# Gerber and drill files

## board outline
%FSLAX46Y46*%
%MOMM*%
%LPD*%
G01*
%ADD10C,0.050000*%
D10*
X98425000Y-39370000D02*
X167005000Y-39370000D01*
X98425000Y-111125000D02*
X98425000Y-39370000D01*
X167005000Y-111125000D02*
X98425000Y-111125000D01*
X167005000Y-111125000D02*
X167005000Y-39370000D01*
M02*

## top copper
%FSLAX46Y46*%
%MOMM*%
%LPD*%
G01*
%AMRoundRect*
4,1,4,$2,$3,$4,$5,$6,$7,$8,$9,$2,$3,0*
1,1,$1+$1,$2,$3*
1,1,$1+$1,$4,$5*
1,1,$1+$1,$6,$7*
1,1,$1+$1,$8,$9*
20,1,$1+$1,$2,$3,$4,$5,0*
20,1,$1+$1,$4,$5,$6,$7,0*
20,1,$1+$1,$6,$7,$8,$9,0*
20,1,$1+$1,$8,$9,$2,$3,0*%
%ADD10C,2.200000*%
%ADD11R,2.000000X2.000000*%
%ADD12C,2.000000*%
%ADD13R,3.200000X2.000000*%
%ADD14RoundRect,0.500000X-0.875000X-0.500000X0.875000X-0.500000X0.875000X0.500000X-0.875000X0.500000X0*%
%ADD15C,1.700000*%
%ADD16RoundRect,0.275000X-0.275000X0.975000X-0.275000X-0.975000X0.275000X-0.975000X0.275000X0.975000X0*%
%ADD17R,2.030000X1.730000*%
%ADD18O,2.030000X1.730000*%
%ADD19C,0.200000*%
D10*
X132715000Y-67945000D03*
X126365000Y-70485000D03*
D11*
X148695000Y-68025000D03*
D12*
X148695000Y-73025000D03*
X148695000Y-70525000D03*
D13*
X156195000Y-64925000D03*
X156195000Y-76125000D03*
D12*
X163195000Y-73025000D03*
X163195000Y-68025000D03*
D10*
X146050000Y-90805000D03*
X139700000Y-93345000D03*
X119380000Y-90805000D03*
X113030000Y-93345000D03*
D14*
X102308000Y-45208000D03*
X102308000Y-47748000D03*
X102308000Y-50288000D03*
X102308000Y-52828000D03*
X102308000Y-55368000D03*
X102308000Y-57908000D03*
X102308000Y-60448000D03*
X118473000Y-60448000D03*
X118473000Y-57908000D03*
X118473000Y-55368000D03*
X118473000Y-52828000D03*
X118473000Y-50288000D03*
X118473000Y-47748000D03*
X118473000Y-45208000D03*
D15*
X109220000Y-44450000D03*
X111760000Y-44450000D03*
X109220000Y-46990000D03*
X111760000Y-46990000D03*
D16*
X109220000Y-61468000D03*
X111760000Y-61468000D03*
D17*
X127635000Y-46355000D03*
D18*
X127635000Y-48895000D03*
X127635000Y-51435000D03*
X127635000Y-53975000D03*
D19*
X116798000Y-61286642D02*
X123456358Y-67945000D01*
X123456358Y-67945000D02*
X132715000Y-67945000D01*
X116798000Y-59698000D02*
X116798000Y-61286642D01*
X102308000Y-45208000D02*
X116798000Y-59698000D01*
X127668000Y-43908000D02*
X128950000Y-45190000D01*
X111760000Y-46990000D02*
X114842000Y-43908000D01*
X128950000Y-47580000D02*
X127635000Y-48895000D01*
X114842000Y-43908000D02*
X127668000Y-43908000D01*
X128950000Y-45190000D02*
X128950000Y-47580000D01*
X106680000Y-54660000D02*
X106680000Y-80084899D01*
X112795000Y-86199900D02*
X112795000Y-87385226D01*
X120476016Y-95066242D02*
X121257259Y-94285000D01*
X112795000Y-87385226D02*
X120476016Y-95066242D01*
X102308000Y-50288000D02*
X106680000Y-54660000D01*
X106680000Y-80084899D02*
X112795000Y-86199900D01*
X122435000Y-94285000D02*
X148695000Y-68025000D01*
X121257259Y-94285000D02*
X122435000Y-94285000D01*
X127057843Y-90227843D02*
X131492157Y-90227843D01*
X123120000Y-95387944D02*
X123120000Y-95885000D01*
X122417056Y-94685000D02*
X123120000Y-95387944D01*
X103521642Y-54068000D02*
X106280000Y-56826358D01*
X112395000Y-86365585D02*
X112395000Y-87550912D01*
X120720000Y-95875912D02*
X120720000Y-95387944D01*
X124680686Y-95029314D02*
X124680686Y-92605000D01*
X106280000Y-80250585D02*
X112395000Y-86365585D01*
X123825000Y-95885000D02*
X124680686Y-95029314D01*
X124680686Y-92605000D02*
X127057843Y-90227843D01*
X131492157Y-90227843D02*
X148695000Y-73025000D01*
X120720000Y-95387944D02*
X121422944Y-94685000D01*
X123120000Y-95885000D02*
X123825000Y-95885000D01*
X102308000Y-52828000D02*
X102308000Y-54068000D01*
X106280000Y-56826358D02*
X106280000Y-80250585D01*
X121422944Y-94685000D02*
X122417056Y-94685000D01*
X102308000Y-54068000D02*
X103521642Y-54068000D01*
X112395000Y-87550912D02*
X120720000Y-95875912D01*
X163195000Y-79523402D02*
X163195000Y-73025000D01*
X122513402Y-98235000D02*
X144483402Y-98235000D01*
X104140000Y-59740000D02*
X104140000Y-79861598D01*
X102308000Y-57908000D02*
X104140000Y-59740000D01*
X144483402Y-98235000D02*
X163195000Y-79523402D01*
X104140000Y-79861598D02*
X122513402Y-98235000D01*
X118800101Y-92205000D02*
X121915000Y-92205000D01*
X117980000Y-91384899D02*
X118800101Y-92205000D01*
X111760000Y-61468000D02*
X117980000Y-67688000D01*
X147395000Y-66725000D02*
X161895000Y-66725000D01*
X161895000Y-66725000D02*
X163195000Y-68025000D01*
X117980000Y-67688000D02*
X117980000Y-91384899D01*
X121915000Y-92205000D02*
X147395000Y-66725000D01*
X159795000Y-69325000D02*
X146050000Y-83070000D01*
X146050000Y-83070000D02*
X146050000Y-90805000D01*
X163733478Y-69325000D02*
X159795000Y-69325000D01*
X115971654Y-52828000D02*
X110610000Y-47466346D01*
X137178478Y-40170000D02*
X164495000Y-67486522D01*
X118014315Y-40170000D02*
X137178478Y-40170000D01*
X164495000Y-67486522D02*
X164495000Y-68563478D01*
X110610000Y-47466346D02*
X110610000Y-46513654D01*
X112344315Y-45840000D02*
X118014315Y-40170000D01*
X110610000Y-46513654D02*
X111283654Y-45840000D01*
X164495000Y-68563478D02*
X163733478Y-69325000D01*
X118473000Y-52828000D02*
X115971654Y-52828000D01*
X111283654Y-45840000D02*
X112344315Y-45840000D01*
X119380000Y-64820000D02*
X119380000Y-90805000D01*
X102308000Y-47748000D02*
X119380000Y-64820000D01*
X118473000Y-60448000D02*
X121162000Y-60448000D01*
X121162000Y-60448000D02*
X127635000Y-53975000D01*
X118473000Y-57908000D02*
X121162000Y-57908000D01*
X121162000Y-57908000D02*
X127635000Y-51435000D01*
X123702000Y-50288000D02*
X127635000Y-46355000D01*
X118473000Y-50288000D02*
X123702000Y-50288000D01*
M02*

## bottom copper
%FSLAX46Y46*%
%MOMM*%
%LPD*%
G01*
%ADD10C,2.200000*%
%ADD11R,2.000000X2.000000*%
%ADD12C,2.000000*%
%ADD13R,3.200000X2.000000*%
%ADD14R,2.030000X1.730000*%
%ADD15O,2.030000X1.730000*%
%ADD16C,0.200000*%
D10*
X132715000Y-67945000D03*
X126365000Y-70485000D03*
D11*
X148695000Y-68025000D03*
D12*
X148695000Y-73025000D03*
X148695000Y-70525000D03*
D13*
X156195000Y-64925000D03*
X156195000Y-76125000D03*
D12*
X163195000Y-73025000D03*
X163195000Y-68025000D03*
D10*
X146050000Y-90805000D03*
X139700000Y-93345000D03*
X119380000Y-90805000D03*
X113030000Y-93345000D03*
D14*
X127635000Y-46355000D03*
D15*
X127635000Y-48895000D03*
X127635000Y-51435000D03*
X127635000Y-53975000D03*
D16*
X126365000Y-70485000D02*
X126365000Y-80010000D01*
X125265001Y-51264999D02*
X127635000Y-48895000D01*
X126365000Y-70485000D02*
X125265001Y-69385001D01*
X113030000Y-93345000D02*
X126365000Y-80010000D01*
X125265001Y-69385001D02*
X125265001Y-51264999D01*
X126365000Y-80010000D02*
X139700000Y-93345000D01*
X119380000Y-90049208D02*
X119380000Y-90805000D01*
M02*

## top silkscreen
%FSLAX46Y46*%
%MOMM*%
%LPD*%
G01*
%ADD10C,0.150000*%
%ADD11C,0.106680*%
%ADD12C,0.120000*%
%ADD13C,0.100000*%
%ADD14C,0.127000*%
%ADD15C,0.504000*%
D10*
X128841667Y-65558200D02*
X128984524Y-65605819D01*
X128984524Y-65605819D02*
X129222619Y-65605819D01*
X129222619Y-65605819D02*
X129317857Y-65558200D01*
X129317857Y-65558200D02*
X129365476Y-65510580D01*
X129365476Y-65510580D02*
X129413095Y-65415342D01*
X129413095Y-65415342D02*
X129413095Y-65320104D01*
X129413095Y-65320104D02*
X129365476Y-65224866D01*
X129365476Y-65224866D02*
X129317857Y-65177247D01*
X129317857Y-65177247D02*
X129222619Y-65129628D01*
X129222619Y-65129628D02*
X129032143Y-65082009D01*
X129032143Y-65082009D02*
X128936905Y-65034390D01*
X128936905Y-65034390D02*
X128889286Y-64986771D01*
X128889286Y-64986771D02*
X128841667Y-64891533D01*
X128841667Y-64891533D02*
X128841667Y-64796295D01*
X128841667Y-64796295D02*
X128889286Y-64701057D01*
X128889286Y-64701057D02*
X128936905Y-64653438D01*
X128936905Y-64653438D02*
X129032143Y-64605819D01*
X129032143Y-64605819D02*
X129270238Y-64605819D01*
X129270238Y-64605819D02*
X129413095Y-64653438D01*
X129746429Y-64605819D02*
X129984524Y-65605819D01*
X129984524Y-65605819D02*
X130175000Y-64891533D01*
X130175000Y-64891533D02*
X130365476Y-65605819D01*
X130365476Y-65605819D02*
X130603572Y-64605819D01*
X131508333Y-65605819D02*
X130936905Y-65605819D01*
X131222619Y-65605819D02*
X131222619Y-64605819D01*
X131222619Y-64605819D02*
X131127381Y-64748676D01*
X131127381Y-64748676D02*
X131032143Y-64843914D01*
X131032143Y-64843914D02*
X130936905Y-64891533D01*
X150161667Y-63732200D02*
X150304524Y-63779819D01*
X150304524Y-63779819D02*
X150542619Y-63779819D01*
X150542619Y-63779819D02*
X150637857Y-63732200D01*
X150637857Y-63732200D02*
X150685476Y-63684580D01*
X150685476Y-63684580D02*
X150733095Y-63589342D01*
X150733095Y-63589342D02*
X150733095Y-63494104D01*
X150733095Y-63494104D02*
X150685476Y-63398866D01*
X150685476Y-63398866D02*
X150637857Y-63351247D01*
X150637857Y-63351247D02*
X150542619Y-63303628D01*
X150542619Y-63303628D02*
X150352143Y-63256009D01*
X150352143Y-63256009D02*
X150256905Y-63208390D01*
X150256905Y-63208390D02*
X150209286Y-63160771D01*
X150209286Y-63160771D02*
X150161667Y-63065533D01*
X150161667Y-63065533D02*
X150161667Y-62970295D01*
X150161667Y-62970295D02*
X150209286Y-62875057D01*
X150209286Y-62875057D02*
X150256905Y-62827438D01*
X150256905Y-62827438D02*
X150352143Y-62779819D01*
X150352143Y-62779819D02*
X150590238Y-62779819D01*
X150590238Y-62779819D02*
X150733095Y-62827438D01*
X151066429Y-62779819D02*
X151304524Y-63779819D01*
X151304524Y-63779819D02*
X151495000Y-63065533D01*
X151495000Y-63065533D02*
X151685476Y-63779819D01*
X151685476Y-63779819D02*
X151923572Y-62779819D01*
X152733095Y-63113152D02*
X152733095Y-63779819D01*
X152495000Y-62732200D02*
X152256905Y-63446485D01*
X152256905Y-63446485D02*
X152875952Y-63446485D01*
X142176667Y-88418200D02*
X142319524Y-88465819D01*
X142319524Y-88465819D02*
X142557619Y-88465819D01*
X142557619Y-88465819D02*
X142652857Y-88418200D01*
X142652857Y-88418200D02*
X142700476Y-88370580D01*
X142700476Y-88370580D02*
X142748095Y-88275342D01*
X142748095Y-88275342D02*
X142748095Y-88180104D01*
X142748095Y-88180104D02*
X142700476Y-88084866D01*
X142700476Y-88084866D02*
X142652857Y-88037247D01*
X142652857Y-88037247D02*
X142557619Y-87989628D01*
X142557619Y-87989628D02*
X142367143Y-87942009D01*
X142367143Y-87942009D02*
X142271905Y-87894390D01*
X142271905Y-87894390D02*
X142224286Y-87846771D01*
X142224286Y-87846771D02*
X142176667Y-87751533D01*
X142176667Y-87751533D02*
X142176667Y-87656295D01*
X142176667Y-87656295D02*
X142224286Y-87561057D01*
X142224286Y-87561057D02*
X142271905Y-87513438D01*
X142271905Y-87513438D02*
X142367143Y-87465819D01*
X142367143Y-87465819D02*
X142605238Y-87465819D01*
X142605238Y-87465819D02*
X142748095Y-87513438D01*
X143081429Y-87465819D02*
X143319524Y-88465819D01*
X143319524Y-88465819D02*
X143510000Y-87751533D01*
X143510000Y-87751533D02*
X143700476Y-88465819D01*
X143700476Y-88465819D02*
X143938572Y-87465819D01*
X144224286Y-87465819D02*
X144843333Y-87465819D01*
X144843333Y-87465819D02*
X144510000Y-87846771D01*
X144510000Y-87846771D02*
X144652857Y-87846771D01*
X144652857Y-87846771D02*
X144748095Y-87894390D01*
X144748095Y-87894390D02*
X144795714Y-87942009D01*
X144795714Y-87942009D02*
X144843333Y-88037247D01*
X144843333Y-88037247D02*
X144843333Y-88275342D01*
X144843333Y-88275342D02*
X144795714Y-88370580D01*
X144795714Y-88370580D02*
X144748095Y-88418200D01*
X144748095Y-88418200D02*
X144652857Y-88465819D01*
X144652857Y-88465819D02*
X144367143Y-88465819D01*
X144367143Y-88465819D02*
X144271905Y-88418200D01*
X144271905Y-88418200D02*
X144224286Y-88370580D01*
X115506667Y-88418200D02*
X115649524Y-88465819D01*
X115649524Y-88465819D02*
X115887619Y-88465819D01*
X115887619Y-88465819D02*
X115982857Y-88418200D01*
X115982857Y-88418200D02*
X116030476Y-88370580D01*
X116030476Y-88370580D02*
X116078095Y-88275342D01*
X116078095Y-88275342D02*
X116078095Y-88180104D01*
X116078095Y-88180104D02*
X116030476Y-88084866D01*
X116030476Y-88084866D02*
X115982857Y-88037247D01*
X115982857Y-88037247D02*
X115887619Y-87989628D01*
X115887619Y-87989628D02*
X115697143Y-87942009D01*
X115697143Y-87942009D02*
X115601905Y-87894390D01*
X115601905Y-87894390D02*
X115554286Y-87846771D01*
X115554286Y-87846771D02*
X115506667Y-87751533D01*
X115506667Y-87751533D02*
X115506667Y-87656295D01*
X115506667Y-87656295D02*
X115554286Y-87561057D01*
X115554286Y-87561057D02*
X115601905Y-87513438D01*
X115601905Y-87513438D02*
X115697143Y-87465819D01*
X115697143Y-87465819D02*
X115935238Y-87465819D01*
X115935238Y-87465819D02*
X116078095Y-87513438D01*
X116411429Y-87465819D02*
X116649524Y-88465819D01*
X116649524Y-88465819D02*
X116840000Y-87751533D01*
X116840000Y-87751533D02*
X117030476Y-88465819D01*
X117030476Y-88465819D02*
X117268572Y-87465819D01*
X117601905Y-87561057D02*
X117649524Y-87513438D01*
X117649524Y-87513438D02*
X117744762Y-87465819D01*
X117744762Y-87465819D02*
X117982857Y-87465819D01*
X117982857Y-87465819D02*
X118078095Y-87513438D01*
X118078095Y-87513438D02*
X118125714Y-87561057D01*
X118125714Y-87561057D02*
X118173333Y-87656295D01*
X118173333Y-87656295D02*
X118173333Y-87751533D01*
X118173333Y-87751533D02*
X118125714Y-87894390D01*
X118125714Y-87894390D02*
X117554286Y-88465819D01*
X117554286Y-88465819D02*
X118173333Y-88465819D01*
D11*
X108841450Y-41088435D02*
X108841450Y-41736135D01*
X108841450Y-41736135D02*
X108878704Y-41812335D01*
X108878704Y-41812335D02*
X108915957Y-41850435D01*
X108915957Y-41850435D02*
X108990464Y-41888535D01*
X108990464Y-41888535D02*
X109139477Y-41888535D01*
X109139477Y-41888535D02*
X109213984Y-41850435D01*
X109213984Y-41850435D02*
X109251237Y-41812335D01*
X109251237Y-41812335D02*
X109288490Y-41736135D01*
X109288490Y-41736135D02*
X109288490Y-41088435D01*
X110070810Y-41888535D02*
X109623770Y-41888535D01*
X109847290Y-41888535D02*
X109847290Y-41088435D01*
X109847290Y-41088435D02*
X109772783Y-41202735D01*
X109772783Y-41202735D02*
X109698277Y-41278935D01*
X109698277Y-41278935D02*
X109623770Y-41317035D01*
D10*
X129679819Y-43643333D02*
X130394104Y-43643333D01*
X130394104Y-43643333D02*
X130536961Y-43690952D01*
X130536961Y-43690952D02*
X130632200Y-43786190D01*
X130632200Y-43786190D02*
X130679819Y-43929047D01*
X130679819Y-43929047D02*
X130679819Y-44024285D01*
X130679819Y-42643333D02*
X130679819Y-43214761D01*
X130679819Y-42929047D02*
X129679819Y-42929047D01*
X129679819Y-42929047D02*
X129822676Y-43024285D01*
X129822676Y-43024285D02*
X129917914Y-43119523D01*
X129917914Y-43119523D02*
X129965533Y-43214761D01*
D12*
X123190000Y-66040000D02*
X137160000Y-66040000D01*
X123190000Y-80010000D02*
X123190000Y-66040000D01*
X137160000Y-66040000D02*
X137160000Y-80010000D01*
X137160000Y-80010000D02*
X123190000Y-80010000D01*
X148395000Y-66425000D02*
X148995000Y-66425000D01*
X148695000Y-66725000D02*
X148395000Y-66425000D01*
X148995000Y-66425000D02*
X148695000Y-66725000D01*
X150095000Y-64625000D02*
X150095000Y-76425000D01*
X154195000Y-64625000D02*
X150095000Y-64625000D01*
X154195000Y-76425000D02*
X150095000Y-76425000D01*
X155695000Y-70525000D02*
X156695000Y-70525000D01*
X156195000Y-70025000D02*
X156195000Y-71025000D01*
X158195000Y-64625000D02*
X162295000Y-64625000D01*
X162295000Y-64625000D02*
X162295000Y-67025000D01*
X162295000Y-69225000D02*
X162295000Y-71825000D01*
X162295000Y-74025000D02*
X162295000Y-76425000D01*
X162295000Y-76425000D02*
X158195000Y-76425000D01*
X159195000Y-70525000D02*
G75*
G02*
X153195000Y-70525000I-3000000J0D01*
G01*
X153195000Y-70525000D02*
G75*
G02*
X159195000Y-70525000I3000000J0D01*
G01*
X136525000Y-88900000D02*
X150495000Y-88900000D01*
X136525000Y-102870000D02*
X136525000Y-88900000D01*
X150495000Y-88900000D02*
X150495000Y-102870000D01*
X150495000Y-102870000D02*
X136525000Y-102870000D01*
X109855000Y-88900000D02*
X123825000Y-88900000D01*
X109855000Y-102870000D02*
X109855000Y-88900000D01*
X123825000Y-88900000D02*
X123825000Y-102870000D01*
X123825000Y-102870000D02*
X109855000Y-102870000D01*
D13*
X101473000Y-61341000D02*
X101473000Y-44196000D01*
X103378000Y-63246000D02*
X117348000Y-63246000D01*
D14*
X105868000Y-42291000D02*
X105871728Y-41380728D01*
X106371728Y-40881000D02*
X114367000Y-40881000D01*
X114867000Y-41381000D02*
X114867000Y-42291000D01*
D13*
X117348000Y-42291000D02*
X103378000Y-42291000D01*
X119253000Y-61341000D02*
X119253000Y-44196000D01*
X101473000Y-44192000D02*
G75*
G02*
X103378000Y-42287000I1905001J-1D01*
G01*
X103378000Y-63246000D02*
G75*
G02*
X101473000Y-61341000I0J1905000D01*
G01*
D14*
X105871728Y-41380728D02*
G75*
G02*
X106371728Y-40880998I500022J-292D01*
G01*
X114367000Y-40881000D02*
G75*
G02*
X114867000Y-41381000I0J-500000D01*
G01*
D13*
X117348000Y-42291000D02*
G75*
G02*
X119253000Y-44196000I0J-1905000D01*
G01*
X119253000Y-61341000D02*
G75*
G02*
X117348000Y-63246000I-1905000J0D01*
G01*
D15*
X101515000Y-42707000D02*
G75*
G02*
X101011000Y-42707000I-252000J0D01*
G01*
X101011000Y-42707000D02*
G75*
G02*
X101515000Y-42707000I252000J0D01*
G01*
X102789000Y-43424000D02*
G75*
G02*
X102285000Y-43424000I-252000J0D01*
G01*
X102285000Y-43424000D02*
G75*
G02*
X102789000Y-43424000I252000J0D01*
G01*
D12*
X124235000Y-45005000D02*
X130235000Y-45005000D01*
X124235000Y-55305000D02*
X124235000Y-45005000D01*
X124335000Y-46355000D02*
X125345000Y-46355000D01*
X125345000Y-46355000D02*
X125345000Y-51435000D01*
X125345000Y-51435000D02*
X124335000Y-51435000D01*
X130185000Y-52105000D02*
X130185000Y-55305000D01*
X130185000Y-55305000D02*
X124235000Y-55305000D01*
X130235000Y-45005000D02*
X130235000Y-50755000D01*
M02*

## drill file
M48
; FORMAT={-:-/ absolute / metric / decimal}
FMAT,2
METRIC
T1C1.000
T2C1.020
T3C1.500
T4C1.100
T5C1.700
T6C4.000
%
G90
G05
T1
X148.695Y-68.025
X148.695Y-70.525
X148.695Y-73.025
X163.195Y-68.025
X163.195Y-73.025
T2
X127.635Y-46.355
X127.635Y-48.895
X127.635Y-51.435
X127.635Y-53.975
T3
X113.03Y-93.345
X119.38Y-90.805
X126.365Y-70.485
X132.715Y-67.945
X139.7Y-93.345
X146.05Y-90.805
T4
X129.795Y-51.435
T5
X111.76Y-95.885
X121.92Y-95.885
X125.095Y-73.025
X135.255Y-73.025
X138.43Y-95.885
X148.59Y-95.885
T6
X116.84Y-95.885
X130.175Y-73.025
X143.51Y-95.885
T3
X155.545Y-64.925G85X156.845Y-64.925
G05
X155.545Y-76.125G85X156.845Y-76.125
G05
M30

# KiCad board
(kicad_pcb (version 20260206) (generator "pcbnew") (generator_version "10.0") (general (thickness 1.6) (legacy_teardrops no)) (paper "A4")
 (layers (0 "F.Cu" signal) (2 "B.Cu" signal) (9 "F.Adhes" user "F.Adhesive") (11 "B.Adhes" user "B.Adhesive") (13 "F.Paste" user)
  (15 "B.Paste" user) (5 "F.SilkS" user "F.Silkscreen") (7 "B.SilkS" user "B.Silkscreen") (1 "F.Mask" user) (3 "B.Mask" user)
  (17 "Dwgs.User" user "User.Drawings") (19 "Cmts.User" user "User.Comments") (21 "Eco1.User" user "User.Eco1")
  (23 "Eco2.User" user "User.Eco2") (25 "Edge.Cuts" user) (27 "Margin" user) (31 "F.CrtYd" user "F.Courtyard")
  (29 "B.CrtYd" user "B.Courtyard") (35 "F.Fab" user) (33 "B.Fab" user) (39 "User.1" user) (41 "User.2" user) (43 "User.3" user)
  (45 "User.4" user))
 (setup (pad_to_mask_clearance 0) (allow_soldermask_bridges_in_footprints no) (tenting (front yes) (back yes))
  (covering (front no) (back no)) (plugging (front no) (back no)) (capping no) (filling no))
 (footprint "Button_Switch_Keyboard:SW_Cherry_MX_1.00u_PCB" (layer "F.Cu") (at 132.715 67.945)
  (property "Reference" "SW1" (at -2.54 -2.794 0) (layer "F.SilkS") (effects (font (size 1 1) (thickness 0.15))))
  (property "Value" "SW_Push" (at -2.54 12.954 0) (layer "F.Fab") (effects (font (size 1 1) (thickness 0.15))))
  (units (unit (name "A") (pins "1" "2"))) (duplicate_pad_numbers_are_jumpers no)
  (fp_line (start -9.525 -1.905) (end 4.445 -1.905) (stroke (width 0.12) (type solid)) (layer "F.SilkS"))
  (fp_line (start -9.525 12.065) (end -9.525 -1.905) (stroke (width 0.12) (type solid)) (layer "F.SilkS"))
  (fp_line (start 4.445 -1.905) (end 4.445 12.065) (stroke (width 0.12) (type solid)) (layer "F.SilkS"))
  (fp_line (start 4.445 12.065) (end -9.525 12.065) (stroke (width 0.12) (type solid)) (layer "F.SilkS"))
  (pad "" np_thru_hole circle (at -7.62 5.08) (size 1.7 1.7) (drill 1.7) (layers "*.Cu" "*.Mask"))
  (pad "" np_thru_hole circle (at -2.54 5.08) (size 4 4) (drill 4) (layers "*.Cu" "*.Mask"))
  (pad "" np_thru_hole circle (at 2.54 5.08) (size 1.7 1.7) (drill 1.7) (layers "*.Cu" "*.Mask"))
  (pad "1" thru_hole circle (at 0 0) (size 2.2 2.2) (drill 1.5) (layers "*.Cu" "*.Mask") (remove_unused_layers no) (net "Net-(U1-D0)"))
  (pad "2" thru_hole circle (at -6.35 2.54) (size 2.2 2.2) (drill 1.5) (layers "*.Cu" "*.Mask") (remove_unused_layers no)
   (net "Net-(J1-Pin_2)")))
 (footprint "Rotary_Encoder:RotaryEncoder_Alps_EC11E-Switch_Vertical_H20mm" (layer "F.Cu") (at 148.695 68.025)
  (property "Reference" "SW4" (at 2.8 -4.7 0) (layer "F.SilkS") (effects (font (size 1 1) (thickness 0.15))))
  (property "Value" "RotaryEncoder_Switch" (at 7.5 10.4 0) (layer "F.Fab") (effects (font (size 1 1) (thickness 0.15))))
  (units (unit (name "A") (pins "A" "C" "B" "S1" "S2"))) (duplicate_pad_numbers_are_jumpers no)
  (fp_line (start -0.3 -1.6) (end 0.3 -1.6) (stroke (width 0.12) (type solid)) (layer "F.SilkS"))
  (fp_line (start 0 -1.3) (end -0.3 -1.6) (stroke (width 0.12) (type solid)) (layer "F.SilkS"))
  (fp_line (start 0.3 -1.6) (end 0 -1.3) (stroke (width 0.12) (type solid)) (layer "F.SilkS"))
  (fp_line (start 1.4 -3.4) (end 1.4 8.4) (stroke (width 0.12) (type solid)) (layer "F.SilkS"))
  (fp_line (start 5.5 -3.4) (end 1.4 -3.4) (stroke (width 0.12) (type solid)) (layer "F.SilkS"))
  (fp_line (start 5.5 8.4) (end 1.4 8.4) (stroke (width 0.12) (type solid)) (layer "F.SilkS"))
  (fp_line (start 7 2.5) (end 8 2.5) (stroke (width 0.12) (type solid)) (layer "F.SilkS"))
  (fp_line (start 7.5 2) (end 7.5 3) (stroke (width 0.12) (type solid)) (layer "F.SilkS"))
  (fp_line (start 9.5 -3.4) (end 13.6 -3.4) (stroke (width 0.12) (type solid)) (layer "F.SilkS"))
  (fp_line (start 13.6 -3.4) (end 13.6 -1) (stroke (width 0.12) (type solid)) (layer "F.SilkS"))
  (fp_line (start 13.6 1.2) (end 13.6 3.8) (stroke (width 0.12) (type solid)) (layer "F.SilkS"))
  (fp_line (start 13.6 6) (end 13.6 8.4) (stroke (width 0.12) (type solid)) (layer "F.SilkS"))
  (fp_line (start 13.6 8.4) (end 9.5 8.4) (stroke (width 0.12) (type solid)) (layer "F.SilkS"))
  (fp_circle (center 7.5 2.5) (end 10.5 2.5) (stroke (width 0.12) (type solid)) (fill no) (layer "F.SilkS"))
  (pad "A" thru_hole rect (at 0 0) (size 2 2) (drill 1) (layers "*.Cu" "*.Mask") (remove_unused_layers no) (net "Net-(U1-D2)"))
  (pad "B" thru_hole circle (at 0 5) (size 2 2) (drill 1) (layers "*.Cu" "*.Mask") (remove_unused_layers no) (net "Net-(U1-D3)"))
  (pad "C" thru_hole circle (at 0 2.5) (size 2 2) (drill 1) (layers "*.Cu" "*.Mask") (remove_unused_layers no)
   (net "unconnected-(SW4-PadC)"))
  (pad "MP" thru_hole rect (at 7.5 -3.1) (size 3.2 2) (drill oval 2.8 1.5) (layers "*.Cu" "*.Mask") (remove_unused_layers no))
  (pad "MP" thru_hole rect (at 7.5 8.1) (size 3.2 2) (drill oval 2.8 1.5) (layers "*.Cu" "*.Mask") (remove_unused_layers no))
  (pad "S1" thru_hole circle (at 14.5 5) (size 2 2) (drill 1) (layers "*.Cu" "*.Mask") (remove_unused_layers no) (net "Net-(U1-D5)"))
  (pad "S2" thru_hole circle (at 14.5 0) (size 2 2) (drill 1) (layers "*.Cu" "*.Mask") (remove_unused_layers no) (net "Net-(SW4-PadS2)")))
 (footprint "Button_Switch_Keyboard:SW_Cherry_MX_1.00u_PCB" (layer "F.Cu") (at 146.05 90.805)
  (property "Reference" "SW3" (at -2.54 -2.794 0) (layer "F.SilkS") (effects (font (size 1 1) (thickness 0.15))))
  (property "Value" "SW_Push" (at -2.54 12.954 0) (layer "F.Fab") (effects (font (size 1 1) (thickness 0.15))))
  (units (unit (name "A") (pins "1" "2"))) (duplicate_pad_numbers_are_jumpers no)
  (fp_line (start -9.525 -1.905) (end 4.445 -1.905) (stroke (width 0.12) (type solid)) (layer "F.SilkS"))
  (fp_line (start -9.525 12.065) (end -9.525 -1.905) (stroke (width 0.12) (type solid)) (layer "F.SilkS"))
  (fp_line (start 4.445 -1.905) (end 4.445 12.065) (stroke (width 0.12) (type solid)) (layer "F.SilkS"))
  (fp_line (start 4.445 12.065) (end -9.525 12.065) (stroke (width 0.12) (type solid)) (layer "F.SilkS"))
  (pad "" np_thru_hole circle (at -7.62 5.08) (size 1.7 1.7) (drill 1.7) (layers "*.Cu" "*.Mask"))
  (pad "" np_thru_hole circle (at -2.54 5.08) (size 4 4) (drill 4) (layers "*.Cu" "*.Mask"))
  (pad "" np_thru_hole circle (at 2.54 5.08) (size 1.7 1.7) (drill 1.7) (layers "*.Cu" "*.Mask"))
  (pad "1" thru_hole circle (at 0 0) (size 2.2 2.2) (drill 1.5) (layers "*.Cu" "*.Mask") (remove_unused_layers no) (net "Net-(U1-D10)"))
  (pad "2" thru_hole circle (at -6.35 2.54) (size 2.2 2.2) (drill 1.5) (layers "*.Cu" "*.Mask") (remove_unused_layers no)
   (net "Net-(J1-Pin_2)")))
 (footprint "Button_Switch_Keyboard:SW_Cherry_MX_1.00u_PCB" (layer "F.Cu") (at 119.38 90.805)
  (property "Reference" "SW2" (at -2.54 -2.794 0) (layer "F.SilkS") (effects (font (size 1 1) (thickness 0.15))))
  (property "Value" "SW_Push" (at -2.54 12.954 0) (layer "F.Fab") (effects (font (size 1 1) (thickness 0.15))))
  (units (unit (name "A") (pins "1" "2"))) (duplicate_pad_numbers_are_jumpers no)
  (fp_line (start -9.525 -1.905) (end 4.445 -1.905) (stroke (width 0.12) (type solid)) (layer "F.SilkS"))
  (fp_line (start -9.525 12.065) (end -9.525 -1.905) (stroke (width 0.12) (type solid)) (layer "F.SilkS"))
  (fp_line (start 4.445 -1.905) (end 4.445 12.065) (stroke (width 0.12) (type solid)) (layer "F.SilkS"))
  (fp_line (start 4.445 12.065) (end -9.525 12.065) (stroke (width 0.12) (type solid)) (layer "F.SilkS"))
  (pad "" np_thru_hole circle (at -7.62 5.08) (size 1.7 1.7) (drill 1.7) (layers "*.Cu" "*.Mask"))
  (pad "" np_thru_hole circle (at -2.54 5.08) (size 4 4) (drill 4) (layers "*.Cu" "*.Mask"))
  (pad "" np_thru_hole circle (at 2.54 5.08) (size 1.7 1.7) (drill 1.7) (layers "*.Cu" "*.Mask"))
  (pad "1" thru_hole circle (at 0 0) (size 2.2 2.2) (drill 1.5) (layers "*.Cu" "*.Mask") (remove_unused_layers no) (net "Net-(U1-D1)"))
  (pad "2" thru_hole circle (at -6.35 2.54) (size 2.2 2.2) (drill 1.5) (layers "*.Cu" "*.Mask") (remove_unused_layers no)
   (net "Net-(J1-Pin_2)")))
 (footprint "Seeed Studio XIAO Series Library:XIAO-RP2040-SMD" (layer "F.Cu") (at 101.473 63.328)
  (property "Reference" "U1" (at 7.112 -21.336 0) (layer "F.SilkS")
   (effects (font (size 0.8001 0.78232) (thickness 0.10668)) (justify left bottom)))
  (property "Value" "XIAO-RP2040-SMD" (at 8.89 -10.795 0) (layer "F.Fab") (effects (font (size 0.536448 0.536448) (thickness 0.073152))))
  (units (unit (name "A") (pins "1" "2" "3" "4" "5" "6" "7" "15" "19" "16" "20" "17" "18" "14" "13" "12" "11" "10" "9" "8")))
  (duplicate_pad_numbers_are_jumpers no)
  (fp_line (start 0 -1.987) (end 0 -19.132) (stroke (width 0.1) (type solid)) (layer "F.SilkS"))
  (fp_line (start 1.905 -0.082) (end 15.875 -0.082) (stroke (width 0.1) (type solid)) (layer "F.SilkS"))
  (fp_line (start 4.395 -21.037) (end 4.398728 -21.947272) (stroke (width 0.127) (type solid)) (layer "F.SilkS"))
  (fp_line (start 4.898728 -22.447) (end 12.894 -22.447) (stroke (width 0.127) (type solid)) (layer "F.SilkS"))
  (fp_line (start 13.394 -21.947) (end 13.394 -21.037) (stroke (width 0.127) (type solid)) (layer "F.SilkS"))
  (fp_line (start 15.875 -21.037) (end 1.905 -21.037) (stroke (width 0.1) (type solid)) (layer "F.SilkS"))
  (fp_line (start 17.78 -1.987) (end 17.78 -19.132) (stroke (width 0.1) (type solid)) (layer "F.SilkS"))
  (fp_arc (start 0 -19.136) (mid 0.557962 -20.483038) (end 1.905 -21.041) (stroke (width 0.1) (type solid)) (layer "F.SilkS"))
  (fp_arc (start 1.905 -0.082) (mid 0.557962 -0.639962) (end 0 -1.987) (stroke (width 0.1) (type solid)) (layer "F.SilkS"))
  (fp_arc (start 4.398728 -21.947272) (mid 4.545276 -22.300644) (end 4.898728 -22.447) (stroke (width 0.127) (type default))
   (layer "F.SilkS"))
  (fp_arc (start 12.894 -22.447) (mid 13.247553 -22.300553) (end 13.394 -21.947) (stroke (width 0.127) (type default)) (layer "F.SilkS"))
  (fp_arc (start 15.875 -21.037) (mid 17.222038 -20.479038) (end 17.78 -19.132) (stroke (width 0.1) (type solid)) (layer "F.SilkS"))
  (fp_arc (start 17.78 -1.987) (mid 17.222038 -0.639962) (end 15.875 -0.082) (stroke (width 0.1) (type solid)) (layer "F.SilkS"))
  (fp_circle (center -0.21 -20.621) (end -0.21 -20.875) (stroke (width 0.5) (type solid)) (fill yes) (layer "F.SilkS"))
  (fp_circle (center 1.064 -19.904) (end 1.064 -20.158) (stroke (width 0.5) (type solid)) (fill yes) (layer "F.SilkS"))
  (pad "1" smd roundrect (at 0.835 -18.12) (size 2.75 2) (layers "F.Cu" "F.Mask" "F.Paste") (roundrect_rratio 0.25) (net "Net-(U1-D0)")
   (solder_mask_margin 0.0508) (thermal_bridge_angle 45))
  (pad "2" smd roundrect (at 0.835 -15.58) (size 2.75 2) (layers "F.Cu" "F.Mask" "F.Paste") (roundrect_rratio 0.25) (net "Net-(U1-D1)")
   (solder_mask_margin 0.0508) (thermal_bridge_angle 45))
  (pad "3" smd roundrect (at 0.835 -13.04) (size 2.75 2) (layers "F.Cu" "F.Mask" "F.Paste") (roundrect_rratio 0.25) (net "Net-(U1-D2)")
   (solder_mask_margin 0.0508) (thermal_bridge_angle 45))
  (pad "4" smd roundrect (at 0.835 -10.5) (size 2.75 2) (layers "F.Cu" "F.Mask" "F.Paste") (roundrect_rratio 0.25) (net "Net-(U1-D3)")
   (solder_mask_margin 0.0508) (thermal_bridge_angle 45))
  (pad "5" smd roundrect (at 0.835 -7.96) (size 2.75 2) (layers "F.Cu" "F.Mask" "F.Paste") (roundrect_rratio 0.25)
   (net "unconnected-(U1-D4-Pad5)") (solder_mask_margin 0.0508) (thermal_bridge_angle 45))
  (pad "6" smd roundrect (at 0.835 -5.42) (size 2.75 2) (layers "F.Cu" "F.Mask" "F.Paste") (roundrect_rratio 0.25) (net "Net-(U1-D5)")
   (solder_mask_margin 0.0508) (thermal_bridge_angle 45))
  (pad "7" smd roundrect (at 0.835 -2.88) (size 2.75 2) (layers "F.Cu" "F.Mask" "F.Paste") (roundrect_rratio 0.25)
   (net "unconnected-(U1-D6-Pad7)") (solder_mask_margin 0.0508) (thermal_bridge_angle 45))
  (pad "8" smd roundrect (at 17 -2.88) (size 2.75 2) (layers "F.Cu" "F.Mask" "F.Paste") (roundrect_rratio 0.25) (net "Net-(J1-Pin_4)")
   (solder_mask_margin 0.0508) (thermal_bridge_angle 45))
  (pad "9" smd roundrect (at 17 -5.42) (size 2.75 2) (layers "F.Cu" "F.Mask" "F.Paste") (roundrect_rratio 0.25) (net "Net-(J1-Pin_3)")
   (solder_mask_margin 0.0508) (thermal_bridge_angle 45))
  (pad "10" smd roundrect (at 17 -7.96) (size 2.75 2) (layers "F.Cu" "F.Mask" "F.Paste") (roundrect_rratio 0.25)
   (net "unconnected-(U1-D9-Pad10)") (solder_mask_margin 0.0508) (thermal_bridge_angle 45))
  (pad "11" smd roundrect (at 17 -10.5) (size 2.75 2) (layers "F.Cu" "F.Mask" "F.Paste") (roundrect_rratio 0.25) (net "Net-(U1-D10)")
   (solder_mask_margin 0.0508) (thermal_bridge_angle 45))
  (pad "12" smd roundrect (at 17 -13.04) (size 2.75 2) (layers "F.Cu" "F.Mask" "F.Paste") (roundrect_rratio 0.25) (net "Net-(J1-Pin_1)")
   (solder_mask_margin 0.0508) (thermal_bridge_angle 45))
  (pad "13" smd roundrect (at 17 -15.58) (size 2.75 2) (layers "F.Cu" "F.Mask" "F.Paste") (roundrect_rratio 0.25)
   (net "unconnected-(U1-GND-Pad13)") (solder_mask_margin 0.0508) (thermal_bridge_angle 45))
  (pad "14" smd roundrect (at 17 -18.12) (size 2.75 2) (layers "F.Cu" "F.Mask" "F.Paste") (roundrect_rratio 0.25)
   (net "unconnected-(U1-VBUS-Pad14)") (solder_mask_margin 0.0508) (thermal_bridge_angle 45))
  (pad "15" smd circle (at 7.747 -18.878) (size 1.7 1.7) (layers "F.Cu" "F.Mask" "F.Paste") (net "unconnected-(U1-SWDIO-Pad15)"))
  (pad "16" smd circle (at 10.287 -18.878) (size 1.7 1.7) (layers "F.Cu" "F.Mask" "F.Paste") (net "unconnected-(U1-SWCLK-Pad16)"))
  (pad "17" smd circle (at 7.747 -16.338) (size 1.7 1.7) (layers "F.Cu" "F.Mask" "F.Paste") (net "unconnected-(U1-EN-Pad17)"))
  (pad "18" smd circle (at 10.287 -16.338) (size 1.7 1.7) (layers "F.Cu" "F.Mask" "F.Paste") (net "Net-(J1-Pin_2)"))
  (pad "19" smd roundrect (at 7.747 -1.86 270) (size 2.5 1.1) (layers "F.Cu" "F.Mask" "F.Paste") (roundrect_rratio 0.25)
   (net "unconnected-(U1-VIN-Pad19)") (thermal_bridge_angle 45))
  (pad "20" smd roundrect (at 10.287 -1.86 270) (size 2.5 1.1) (layers "F.Cu" "F.Mask" "F.Paste") (roundrect_rratio 0.25)
   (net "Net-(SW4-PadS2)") (thermal_bridge_angle 45)))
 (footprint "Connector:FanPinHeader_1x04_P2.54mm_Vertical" (layer "F.Cu") (at 127.635 46.355 -90)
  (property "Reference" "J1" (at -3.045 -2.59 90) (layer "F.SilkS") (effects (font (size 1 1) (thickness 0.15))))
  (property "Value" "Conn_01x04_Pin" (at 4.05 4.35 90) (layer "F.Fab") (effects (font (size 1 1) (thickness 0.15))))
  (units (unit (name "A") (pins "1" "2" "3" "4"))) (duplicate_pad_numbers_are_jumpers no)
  (fp_line (start -1.35 3.4) (end -1.35 -2.6) (stroke (width 0.12) (type solid)) (layer "F.SilkS"))
  (fp_line (start 8.95 3.4) (end -1.35 3.4) (stroke (width 0.12) (type solid)) (layer "F.SilkS"))
  (fp_line (start 0 3.3) (end 0 2.29) (stroke (width 0.12) (type solid)) (layer "F.SilkS"))
  (fp_line (start 0 2.29) (end 5.08 2.29) (stroke (width 0.12) (type solid)) (layer "F.SilkS"))
  (fp_line (start 5.08 2.29) (end 5.08 3.3) (stroke (width 0.12) (type solid)) (layer "F.SilkS"))
  (fp_line (start 5.75 -2.55) (end 8.95 -2.55) (stroke (width 0.12) (type solid)) (layer "F.SilkS"))
  (fp_line (start 8.95 -2.55) (end 8.95 3.4) (stroke (width 0.12) (type solid)) (layer "F.SilkS"))
  (fp_line (start -1.35 -2.6) (end 4.4 -2.6) (stroke (width 0.12) (type solid)) (layer "F.SilkS"))
  (pad "" np_thru_hole circle (at 5.08 -2.16) (size 1.1 1.1) (drill 1.1) (layers "*.Cu" "*.Mask"))
  (pad "1" thru_hole rect (at 0 0) (size 2.03 1.73) (drill 1.02) (layers "*.Cu" "*.Mask") (remove_unused_layers no) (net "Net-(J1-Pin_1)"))
  (pad "2" thru_hole oval (at 2.54 0) (size 2.03 1.73) (drill 1.02) (layers "*.Cu" "*.Mask") (remove_unused_layers no)
   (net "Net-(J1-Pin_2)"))
  (pad "3" thru_hole oval (at 5.08 0) (size 2.03 1.73) (drill 1.02) (layers "*.Cu" "*.Mask") (remove_unused_layers no)
   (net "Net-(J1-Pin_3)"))
  (pad "4" thru_hole oval (at 7.62 0) (size 2.03 1.73) (drill 1.02) (layers "*.Cu" "*.Mask") (remove_unused_layers no)
   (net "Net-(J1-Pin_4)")))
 (gr_line (start 98.425 39.37) (end 167.005 39.37) (stroke (width 0.05) (type default)) (layer "Edge.Cuts"))
 (gr_line (start 98.425 111.125) (end 98.425 39.37) (stroke (width 0.05) (type default)) (layer "Edge.Cuts"))
 (gr_line (start 167.005 111.125) (end 98.425 111.125) (stroke (width 0.05) (type default)) (layer "Edge.Cuts"))
 (gr_line (start 167.005 111.125) (end 167.005 39.37) (stroke (width 0.05) (type default)) (layer "Edge.Cuts"))
 (segment (start 116.798 61.286642) (end 123.456358 67.945) (width 0.2) (layer "F.Cu") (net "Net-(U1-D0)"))
 (segment (start 123.456358 67.945) (end 132.715 67.945) (width 0.2) (layer "F.Cu") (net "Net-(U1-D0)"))
 (segment (start 116.798 59.698) (end 116.798 61.286642) (width 0.2) (layer "F.Cu") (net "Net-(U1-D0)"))
 (segment (start 102.308 45.208) (end 116.798 59.698) (width 0.2) (layer "F.Cu") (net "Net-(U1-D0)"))
 (segment (start 127.668 43.908) (end 128.95 45.19) (width 0.2) (layer "F.Cu") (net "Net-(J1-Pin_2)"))
 (segment (start 111.76 46.99) (end 114.842 43.908) (width 0.2) (layer "F.Cu") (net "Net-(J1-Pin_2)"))
 (segment (start 128.95 47.58) (end 127.635 48.895) (width 0.2) (layer "F.Cu") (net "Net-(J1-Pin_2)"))
 (segment (start 114.842 43.908) (end 127.668 43.908) (width 0.2) (layer "F.Cu") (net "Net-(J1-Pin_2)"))
 (segment (start 128.95 45.19) (end 128.95 47.58) (width 0.2) (layer "F.Cu") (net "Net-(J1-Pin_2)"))
 (segment (start 126.365 70.485) (end 126.365 80.01) (width 0.2) (layer "B.Cu") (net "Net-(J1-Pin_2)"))
 (segment (start 125.265001 51.264999) (end 127.635 48.895) (width 0.2) (layer "B.Cu") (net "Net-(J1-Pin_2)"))
 (segment (start 126.365 70.485) (end 125.265001 69.385001) (width 0.2) (layer "B.Cu") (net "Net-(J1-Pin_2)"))
 (segment (start 113.03 93.345) (end 126.365 80.01) (width 0.2) (layer "B.Cu") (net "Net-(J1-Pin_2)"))
 (segment (start 125.265001 69.385001) (end 125.265001 51.264999) (width 0.2) (layer "B.Cu") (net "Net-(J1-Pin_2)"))
 (segment (start 126.365 80.01) (end 139.7 93.345) (width 0.2) (layer "B.Cu") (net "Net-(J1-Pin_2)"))
 (segment (start 106.68 54.66) (end 106.68 80.084899) (width 0.2) (layer "F.Cu") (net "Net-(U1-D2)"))
 (segment (start 112.795 86.1999) (end 112.795 87.385226) (width 0.2) (layer "F.Cu") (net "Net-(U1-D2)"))
 (segment (start 120.476016 95.066242) (end 121.257259 94.285) (width 0.2) (layer "F.Cu") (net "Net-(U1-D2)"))
 (segment (start 112.795 87.385226) (end 120.476016 95.066242) (width 0.2) (layer "F.Cu") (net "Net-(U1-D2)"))
 (segment (start 102.308 50.288) (end 106.68 54.66) (width 0.2) (layer "F.Cu") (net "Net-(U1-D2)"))
 (segment (start 106.68 80.084899) (end 112.795 86.1999) (width 0.2) (layer "F.Cu") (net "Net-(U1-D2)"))
 (segment (start 122.435 94.285) (end 148.695 68.025) (width 0.2) (layer "F.Cu") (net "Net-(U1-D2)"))
 (segment (start 121.257259 94.285) (end 122.435 94.285) (width 0.2) (layer "F.Cu") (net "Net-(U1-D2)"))
 (segment (start 127.057843 90.227843) (end 131.492157 90.227843) (width 0.2) (layer "F.Cu") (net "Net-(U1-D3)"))
 (segment (start 123.12 95.387944) (end 123.12 95.885) (width 0.2) (layer "F.Cu") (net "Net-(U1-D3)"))
 (segment (start 122.417056 94.685) (end 123.12 95.387944) (width 0.2) (layer "F.Cu") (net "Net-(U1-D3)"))
 (segment (start 103.521642 54.068) (end 106.28 56.826358) (width 0.2) (layer "F.Cu") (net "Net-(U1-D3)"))
 (segment (start 112.395 86.365585) (end 112.395 87.550912) (width 0.2) (layer "F.Cu") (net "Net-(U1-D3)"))
 (segment (start 120.72 95.875912) (end 120.72 95.387944) (width 0.2) (layer "F.Cu") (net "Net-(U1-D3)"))
 (segment (start 124.680686 95.029314) (end 124.680686 92.605) (width 0.2) (layer "F.Cu") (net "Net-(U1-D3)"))
 (segment (start 106.28 80.250585) (end 112.395 86.365585) (width 0.2) (layer "F.Cu") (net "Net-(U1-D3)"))
 (segment (start 123.825 95.885) (end 124.680686 95.029314) (width 0.2) (layer "F.Cu") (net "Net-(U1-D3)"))
 (segment (start 124.680686 92.605) (end 127.057843 90.227843) (width 0.2) (layer "F.Cu") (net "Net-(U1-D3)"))
 (segment (start 131.492157 90.227843) (end 148.695 73.025) (width 0.2) (layer "F.Cu") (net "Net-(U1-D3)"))
 (segment (start 120.72 95.387944) (end 121.422944 94.685) (width 0.2) (layer "F.Cu") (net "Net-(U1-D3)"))
 (segment (start 123.12 95.885) (end 123.825 95.885) (width 0.2) (layer "F.Cu") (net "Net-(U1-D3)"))
 (segment (start 102.308 52.828) (end 102.308 54.068) (width 0.2) (layer "F.Cu") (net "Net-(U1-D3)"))
 (segment (start 106.28 56.826358) (end 106.28 80.250585) (width 0.2) (layer "F.Cu") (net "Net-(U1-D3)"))
 (segment (start 121.422944 94.685) (end 122.417056 94.685) (width 0.2) (layer "F.Cu") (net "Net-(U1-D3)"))
 (segment (start 102.308 54.068) (end 103.521642 54.068) (width 0.2) (layer "F.Cu") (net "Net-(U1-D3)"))
 (segment (start 112.395 87.550912) (end 120.72 95.875912) (width 0.2) (layer "F.Cu") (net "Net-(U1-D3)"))
 (segment (start 163.195 79.523402) (end 163.195 73.025) (width 0.2) (layer "F.Cu") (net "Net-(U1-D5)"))
 (segment (start 122.513402 98.235) (end 144.483402 98.235) (width 0.2) (layer "F.Cu") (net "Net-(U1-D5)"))
 (segment (start 104.14 59.74) (end 104.14 79.861598) (width 0.2) (layer "F.Cu") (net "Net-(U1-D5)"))
 (segment (start 102.308 57.908) (end 104.14 59.74) (width 0.2) (layer "F.Cu") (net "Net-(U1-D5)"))
 (segment (start 144.483402 98.235) (end 163.195 79.523402) (width 0.2) (layer "F.Cu") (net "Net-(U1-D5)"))
 (segment (start 104.14 79.861598) (end 122.513402 98.235) (width 0.2) (layer "F.Cu") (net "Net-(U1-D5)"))
 (segment (start 118.800101 92.205) (end 121.915 92.205) (width 0.2) (layer "F.Cu") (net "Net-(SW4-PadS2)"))
 (segment (start 117.98 91.384899) (end 118.800101 92.205) (width 0.2) (layer "F.Cu") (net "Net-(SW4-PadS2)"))
 (segment (start 111.76 61.468) (end 117.98 67.688) (width 0.2) (layer "F.Cu") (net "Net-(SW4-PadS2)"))
 (segment (start 147.395 66.725) (end 161.895 66.725) (width 0.2) (layer "F.Cu") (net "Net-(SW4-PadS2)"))
 (segment (start 161.895 66.725) (end 163.195 68.025) (width 0.2) (layer "F.Cu") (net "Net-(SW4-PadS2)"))
 (segment (start 117.98 67.688) (end 117.98 91.384899) (width 0.2) (layer "F.Cu") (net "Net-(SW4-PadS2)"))
 (segment (start 121.915 92.205) (end 147.395 66.725) (width 0.2) (layer "F.Cu") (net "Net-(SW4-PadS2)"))
 (segment (start 159.795 69.325) (end 146.05 83.07) (width 0.2) (layer "F.Cu") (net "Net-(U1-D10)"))
 (segment (start 146.05 83.07) (end 146.05 90.805) (width 0.2) (layer "F.Cu") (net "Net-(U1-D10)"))
 (segment (start 163.733478 69.325) (end 159.795 69.325) (width 0.2) (layer "F.Cu") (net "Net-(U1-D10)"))
 (segment (start 115.971654 52.828) (end 110.61 47.466346) (width 0.2) (layer "F.Cu") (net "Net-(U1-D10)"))
 (segment (start 137.178478 40.17) (end 164.495 67.486522) (width 0.2) (layer "F.Cu") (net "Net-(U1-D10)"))
 (segment (start 118.014315 40.17) (end 137.178478 40.17) (width 0.2) (layer "F.Cu") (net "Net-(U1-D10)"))
 (segment (start 164.495 67.486522) (end 164.495 68.563478) (width 0.2) (layer "F.Cu") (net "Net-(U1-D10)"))
 (segment (start 110.61 47.466346) (end 110.61 46.513654) (width 0.2) (layer "F.Cu") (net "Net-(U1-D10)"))
 (segment (start 112.344315 45.84) (end 118.014315 40.17) (width 0.2) (layer "F.Cu") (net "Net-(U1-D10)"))
 (segment (start 110.61 46.513654) (end 111.283654 45.84) (width 0.2) (layer "F.Cu") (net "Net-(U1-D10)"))
 (segment (start 164.495 68.563478) (end 163.733478 69.325) (width 0.2) (layer "F.Cu") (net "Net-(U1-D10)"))
 (segment (start 118.473 52.828) (end 115.971654 52.828) (width 0.2) (layer "F.Cu") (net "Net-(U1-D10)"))
 (segment (start 111.283654 45.84) (end 112.344315 45.84) (width 0.2) (layer "F.Cu") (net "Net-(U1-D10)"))
 (segment (start 119.38 64.82) (end 119.38 90.805) (width 0.2) (layer "F.Cu") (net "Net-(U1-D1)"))
 (segment (start 102.308 47.748) (end 119.38 64.82) (width 0.2) (layer "F.Cu") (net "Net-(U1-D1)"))
 (segment (start 119.38 90.049208) (end 119.38 90.805) (width 0.2) (layer "B.Cu") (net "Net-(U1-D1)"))
 (segment (start 118.473 60.448) (end 121.162 60.448) (width 0.2) (layer "F.Cu") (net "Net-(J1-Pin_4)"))
 (segment (start 121.162 60.448) (end 127.635 53.975) (width 0.2) (layer "F.Cu") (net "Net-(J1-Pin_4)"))
 (segment (start 118.473 57.908) (end 121.162 57.908) (width 0.2) (layer "F.Cu") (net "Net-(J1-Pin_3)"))
 (segment (start 121.162 57.908) (end 127.635 51.435) (width 0.2) (layer "F.Cu") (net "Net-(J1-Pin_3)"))
 (segment (start 123.702 50.288) (end 127.635 46.355) (width 0.2) (layer "F.Cu") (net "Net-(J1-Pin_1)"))
 (segment (start 118.473 50.288) (end 123.702 50.288) (width 0.2) (layer "F.Cu") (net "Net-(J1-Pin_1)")))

